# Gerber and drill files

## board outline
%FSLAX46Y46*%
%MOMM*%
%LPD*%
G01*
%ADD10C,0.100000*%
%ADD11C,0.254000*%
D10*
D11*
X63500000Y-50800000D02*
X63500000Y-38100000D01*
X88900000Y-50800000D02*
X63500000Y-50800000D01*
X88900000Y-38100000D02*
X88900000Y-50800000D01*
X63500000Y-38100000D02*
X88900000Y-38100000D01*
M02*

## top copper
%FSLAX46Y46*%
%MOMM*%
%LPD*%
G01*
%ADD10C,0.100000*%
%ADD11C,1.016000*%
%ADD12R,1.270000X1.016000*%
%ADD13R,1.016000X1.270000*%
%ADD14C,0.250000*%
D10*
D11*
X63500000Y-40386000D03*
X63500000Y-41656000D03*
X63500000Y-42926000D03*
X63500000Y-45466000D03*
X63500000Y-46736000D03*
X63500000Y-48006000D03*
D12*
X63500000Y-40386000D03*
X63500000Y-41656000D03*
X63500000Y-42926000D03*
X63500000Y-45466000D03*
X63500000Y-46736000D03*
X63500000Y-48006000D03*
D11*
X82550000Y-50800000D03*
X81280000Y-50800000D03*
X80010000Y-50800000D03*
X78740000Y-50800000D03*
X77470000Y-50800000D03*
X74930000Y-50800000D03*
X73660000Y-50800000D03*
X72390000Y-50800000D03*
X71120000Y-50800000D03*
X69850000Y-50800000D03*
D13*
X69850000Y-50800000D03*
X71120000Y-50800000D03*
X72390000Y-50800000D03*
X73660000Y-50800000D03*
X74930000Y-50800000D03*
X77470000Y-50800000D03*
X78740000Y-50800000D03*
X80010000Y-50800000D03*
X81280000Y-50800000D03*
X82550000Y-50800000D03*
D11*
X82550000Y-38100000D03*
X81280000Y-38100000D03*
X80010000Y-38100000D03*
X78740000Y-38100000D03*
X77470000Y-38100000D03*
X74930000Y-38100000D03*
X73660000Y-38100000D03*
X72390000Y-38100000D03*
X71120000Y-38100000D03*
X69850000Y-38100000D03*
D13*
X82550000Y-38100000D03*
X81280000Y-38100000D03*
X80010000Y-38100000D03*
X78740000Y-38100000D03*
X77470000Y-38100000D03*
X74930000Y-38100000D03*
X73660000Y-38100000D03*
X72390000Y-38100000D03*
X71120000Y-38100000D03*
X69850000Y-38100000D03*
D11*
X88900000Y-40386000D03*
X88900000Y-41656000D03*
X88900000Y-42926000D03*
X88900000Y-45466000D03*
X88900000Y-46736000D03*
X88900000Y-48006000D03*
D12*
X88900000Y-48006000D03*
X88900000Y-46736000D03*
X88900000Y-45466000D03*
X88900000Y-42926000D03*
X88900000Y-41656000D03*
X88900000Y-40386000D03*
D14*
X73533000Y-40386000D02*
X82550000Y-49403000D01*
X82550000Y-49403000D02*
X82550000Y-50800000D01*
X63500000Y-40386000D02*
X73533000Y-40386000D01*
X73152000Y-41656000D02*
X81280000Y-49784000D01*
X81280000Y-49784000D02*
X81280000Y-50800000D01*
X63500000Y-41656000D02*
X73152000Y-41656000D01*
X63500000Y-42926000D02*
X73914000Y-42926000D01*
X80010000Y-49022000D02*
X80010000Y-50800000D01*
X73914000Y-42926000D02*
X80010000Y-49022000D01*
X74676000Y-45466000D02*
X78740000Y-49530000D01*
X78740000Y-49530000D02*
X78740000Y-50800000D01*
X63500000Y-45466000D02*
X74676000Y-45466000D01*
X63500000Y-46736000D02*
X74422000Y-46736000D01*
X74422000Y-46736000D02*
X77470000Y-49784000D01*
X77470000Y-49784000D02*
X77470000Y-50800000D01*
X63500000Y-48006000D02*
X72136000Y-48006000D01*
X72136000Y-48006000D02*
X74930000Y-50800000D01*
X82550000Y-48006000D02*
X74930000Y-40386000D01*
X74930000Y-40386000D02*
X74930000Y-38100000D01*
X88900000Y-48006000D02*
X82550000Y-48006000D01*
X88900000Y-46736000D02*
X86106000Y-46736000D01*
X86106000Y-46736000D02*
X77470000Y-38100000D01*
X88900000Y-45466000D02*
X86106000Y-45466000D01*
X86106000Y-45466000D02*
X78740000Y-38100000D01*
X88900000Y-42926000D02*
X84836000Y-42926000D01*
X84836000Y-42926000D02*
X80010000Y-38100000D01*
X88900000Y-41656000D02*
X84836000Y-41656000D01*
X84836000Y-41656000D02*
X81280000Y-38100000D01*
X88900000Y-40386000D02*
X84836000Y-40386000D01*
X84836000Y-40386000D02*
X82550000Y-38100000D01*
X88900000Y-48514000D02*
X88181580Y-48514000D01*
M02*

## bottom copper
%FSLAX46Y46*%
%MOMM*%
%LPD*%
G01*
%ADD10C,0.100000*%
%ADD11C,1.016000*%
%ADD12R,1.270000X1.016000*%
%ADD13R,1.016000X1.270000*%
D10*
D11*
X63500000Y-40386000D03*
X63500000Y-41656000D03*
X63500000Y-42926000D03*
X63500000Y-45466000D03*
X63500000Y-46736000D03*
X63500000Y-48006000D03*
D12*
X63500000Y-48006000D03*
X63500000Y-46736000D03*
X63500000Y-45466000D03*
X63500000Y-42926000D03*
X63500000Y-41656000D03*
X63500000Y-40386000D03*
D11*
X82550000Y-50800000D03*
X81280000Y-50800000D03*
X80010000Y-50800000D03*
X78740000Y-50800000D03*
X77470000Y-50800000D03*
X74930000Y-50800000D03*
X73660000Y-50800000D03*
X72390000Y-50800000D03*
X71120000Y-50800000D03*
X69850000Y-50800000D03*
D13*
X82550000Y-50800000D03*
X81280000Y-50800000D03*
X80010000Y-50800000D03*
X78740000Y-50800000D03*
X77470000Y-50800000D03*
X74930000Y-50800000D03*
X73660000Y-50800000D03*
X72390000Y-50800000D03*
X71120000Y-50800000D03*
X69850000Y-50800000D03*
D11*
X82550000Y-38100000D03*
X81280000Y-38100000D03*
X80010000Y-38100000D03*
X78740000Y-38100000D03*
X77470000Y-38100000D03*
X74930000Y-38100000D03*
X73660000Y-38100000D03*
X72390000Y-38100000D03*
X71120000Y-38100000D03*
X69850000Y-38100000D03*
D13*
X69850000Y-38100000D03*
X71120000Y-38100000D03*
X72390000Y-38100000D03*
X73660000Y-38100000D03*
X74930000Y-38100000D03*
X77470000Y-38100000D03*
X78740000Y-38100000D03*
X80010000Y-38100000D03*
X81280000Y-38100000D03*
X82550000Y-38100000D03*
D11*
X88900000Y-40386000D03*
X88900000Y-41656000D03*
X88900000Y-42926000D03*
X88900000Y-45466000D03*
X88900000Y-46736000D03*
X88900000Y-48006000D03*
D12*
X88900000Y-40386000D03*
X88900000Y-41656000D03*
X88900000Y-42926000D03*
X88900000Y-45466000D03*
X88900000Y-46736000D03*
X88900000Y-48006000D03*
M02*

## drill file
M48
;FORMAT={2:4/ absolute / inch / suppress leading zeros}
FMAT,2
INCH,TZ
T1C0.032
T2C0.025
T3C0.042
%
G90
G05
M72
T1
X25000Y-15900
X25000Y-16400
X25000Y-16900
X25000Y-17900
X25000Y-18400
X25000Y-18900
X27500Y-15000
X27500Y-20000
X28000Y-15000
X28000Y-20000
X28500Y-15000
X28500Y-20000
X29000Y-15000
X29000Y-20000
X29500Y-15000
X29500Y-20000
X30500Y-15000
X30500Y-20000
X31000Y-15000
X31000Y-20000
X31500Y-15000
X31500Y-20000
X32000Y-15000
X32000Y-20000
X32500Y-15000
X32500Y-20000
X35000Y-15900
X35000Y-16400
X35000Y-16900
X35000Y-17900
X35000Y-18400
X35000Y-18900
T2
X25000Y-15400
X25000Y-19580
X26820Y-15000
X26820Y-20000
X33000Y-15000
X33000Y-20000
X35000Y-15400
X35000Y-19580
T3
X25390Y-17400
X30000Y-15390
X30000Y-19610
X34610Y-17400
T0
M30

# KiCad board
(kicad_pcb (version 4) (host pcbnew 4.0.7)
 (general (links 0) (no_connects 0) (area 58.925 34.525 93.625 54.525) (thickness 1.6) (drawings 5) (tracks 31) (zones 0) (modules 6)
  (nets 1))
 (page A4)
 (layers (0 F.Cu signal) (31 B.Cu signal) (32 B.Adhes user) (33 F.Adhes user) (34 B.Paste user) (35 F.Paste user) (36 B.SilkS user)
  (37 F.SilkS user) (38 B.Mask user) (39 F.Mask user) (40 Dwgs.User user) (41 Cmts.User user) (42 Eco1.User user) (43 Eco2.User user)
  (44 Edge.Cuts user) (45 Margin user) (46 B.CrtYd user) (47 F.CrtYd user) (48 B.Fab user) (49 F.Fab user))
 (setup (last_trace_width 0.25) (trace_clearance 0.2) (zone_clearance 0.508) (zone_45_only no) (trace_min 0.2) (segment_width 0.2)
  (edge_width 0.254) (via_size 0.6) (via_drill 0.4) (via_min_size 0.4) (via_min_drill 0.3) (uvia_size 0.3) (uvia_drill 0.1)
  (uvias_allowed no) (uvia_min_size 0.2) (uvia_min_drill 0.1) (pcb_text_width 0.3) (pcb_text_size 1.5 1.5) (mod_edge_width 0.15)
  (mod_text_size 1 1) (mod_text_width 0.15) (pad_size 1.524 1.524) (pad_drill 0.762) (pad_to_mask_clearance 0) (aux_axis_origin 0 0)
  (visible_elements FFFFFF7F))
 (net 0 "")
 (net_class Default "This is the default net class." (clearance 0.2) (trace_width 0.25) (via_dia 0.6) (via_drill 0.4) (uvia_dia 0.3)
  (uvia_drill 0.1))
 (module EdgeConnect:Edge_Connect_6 (layer F.Cu) (at 63.5 44.196 90)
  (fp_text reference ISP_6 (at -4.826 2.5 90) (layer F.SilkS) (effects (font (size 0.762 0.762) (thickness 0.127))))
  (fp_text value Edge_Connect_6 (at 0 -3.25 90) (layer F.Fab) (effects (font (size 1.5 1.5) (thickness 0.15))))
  (pad 1 thru_hole circle (at 3.81 0 90) (size 1.016 1.016) (drill 0.8128) (layers *.Cu *.Mask))
  (pad "" np_thru_hole circle (at 0 0.9906 90) (size 1.0668 1.0668) (drill 1.0668) (layers *.Cu))
  (pad 2 thru_hole circle (at 2.54 0 90) (size 1.016 1.016) (drill 0.8128) (layers *.Cu *.Mask))
  (pad 3 thru_hole circle (at 1.27 0 90) (size 1.016 1.016) (drill 0.8128) (layers *.Cu *.Mask))
  (pad 4 thru_hole circle (at -1.27 0 90) (size 1.016 1.016) (drill 0.8128) (layers *.Cu *.Mask))
  (pad 5 thru_hole circle (at -2.54 0 90) (size 1.016 1.016) (drill 0.8128) (layers *.Cu *.Mask))
  (pad 6 thru_hole circle (at -3.81 0 90) (size 1.016 1.016) (drill 0.8128) (layers *.Cu *.Mask))
  (pad "" np_thru_hole circle (at -5.5372 0 90) (size 0.635 0.635) (drill 0.635) (layers *.Cu))
  (pad "" np_thru_hole circle (at 5.08 0 90) (size 0.635 0.635) (drill 0.635) (layers *.Cu))
  (pad 1 smd rect (at 3.81 0 90) (size 1.016 1.27) (layers F.Cu F.Mask))
  (pad 2 smd rect (at 2.54 0 90) (size 1.016 1.27) (layers F.Cu F.Mask))
  (pad 3 smd rect (at 1.27 0 90) (size 1.016 1.27) (layers F.Cu F.Mask))
  (pad 4 smd rect (at -1.27 0 90) (size 1.016 1.27) (layers F.Cu F.Mask))
  (pad 5 smd rect (at -2.54 0 90) (size 1.016 1.27) (layers F.Cu F.Mask))
  (pad 6 smd rect (at -3.81 0 90) (size 1.016 1.27) (layers F.Cu F.Mask))
  (pad 6 smd rect (at -3.81 0 90) (size 1.016 1.27) (layers B.Cu B.Mask))
  (pad 5 smd rect (at -2.54 0 90) (size 1.016 1.27) (layers B.Cu B.Mask))
  (pad 4 smd rect (at -1.27 0 90) (size 1.016 1.27) (layers B.Cu B.Mask))
  (pad 3 smd rect (at 1.27 0 90) (size 1.016 1.27) (layers B.Cu B.Mask))
  (pad 2 smd rect (at 2.54 0 90) (size 1.016 1.27) (layers B.Cu B.Mask))
  (pad 1 smd rect (at 3.81 0 90) (size 1.016 1.27) (layers B.Cu B.Mask)))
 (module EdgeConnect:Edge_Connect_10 (layer B.Cu) (at 76.2 50.8)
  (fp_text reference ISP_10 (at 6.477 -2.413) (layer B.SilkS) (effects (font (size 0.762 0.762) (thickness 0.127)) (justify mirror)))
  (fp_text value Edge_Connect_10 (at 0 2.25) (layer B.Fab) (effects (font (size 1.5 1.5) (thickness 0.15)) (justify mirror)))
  (pad 1 thru_hole circle (at 6.35 0) (size 1.016 1.016) (drill 0.8128) (layers *.Cu *.Mask))
  (pad "" np_thru_hole circle (at 0 -0.9906) (size 1.0668 1.0668) (drill 1.0668) (layers *.Cu))
  (pad 2 thru_hole circle (at 5.08 0) (size 1.016 1.016) (drill 0.8128) (layers *.Cu *.Mask))
  (pad 3 thru_hole circle (at 3.81 0) (size 1.016 1.016) (drill 0.8128) (layers *.Cu *.Mask))
  (pad 4 thru_hole circle (at 2.54 0) (size 1.016 1.016) (drill 0.8128) (layers *.Cu *.Mask))
  (pad 5 thru_hole circle (at 1.27 0) (size 1.016 1.016) (drill 0.8128) (layers *.Cu *.Mask))
  (pad 6 thru_hole circle (at -1.27 0) (size 1.016 1.016) (drill 0.8128) (layers *.Cu *.Mask))
  (pad "" np_thru_hole circle (at -8.0772 0) (size 0.635 0.635) (drill 0.635) (layers *.Cu))
  (pad "" np_thru_hole circle (at 7.62 0) (size 0.635 0.635) (drill 0.635) (layers *.Cu))
  (pad 7 thru_hole circle (at -2.54 0) (size 1.016 1.016) (drill 0.8128) (layers *.Cu *.Mask))
  (pad 8 thru_hole circle (at -3.81 0) (size 1.016 1.016) (drill 0.8128) (layers *.Cu *.Mask))
  (pad 9 thru_hole circle (at -5.08 0) (size 1.016 1.016) (drill 0.8128) (layers *.Cu *.Mask))
  (pad 10 thru_hole circle (at -6.35 0) (size 1.016 1.016) (drill 0.8128) (layers *.Cu *.Mask))
  (pad 1 smd rect (at 6.35 0) (size 1.016 1.27) (layers B.Cu B.Mask))
  (pad 2 smd rect (at 5.08 0) (size 1.016 1.27) (layers B.Cu B.Mask))
  (pad 3 smd rect (at 3.81 0) (size 1.016 1.27) (layers B.Cu B.Mask))
  (pad 4 smd rect (at 2.54 0) (size 1.016 1.27) (layers B.Cu B.Mask))
  (pad 5 smd rect (at 1.27 0) (size 1.016 1.27) (layers B.Cu B.Mask))
  (pad 5 smd rect (at -1.27 0) (size 1.016 1.27) (layers B.Cu B.Mask))
  (pad 7 smd rect (at -2.54 0) (size 1.016 1.27) (layers B.Cu B.Mask))
  (pad 8 smd rect (at -3.81 0) (size 1.016 1.27) (layers B.Cu B.Mask))
  (pad 9 smd rect (at -5.08 0) (size 1.016 1.27) (layers B.Cu B.Mask))
  (pad 10 smd rect (at -6.35 0) (size 1.016 1.27) (layers B.Cu B.Mask))
  (pad 10 smd rect (at -6.35 0) (size 1.016 1.27) (layers F.Cu F.Mask))
  (pad 9 smd rect (at -5.08 0) (size 1.016 1.27) (layers F.Cu F.Mask))
  (pad 8 smd rect (at -3.81 0) (size 1.016 1.27) (layers F.Cu F.Mask))
  (pad 7 smd rect (at -2.54 0) (size 1.016 1.27) (layers F.Cu F.Mask))
  (pad 5 smd rect (at -1.27 0) (size 1.016 1.27) (layers F.Cu F.Mask))
  (pad 5 smd rect (at 1.27 0) (size 1.016 1.27) (layers F.Cu F.Mask))
  (pad 4 smd rect (at 2.54 0) (size 1.016 1.27) (layers F.Cu F.Mask))
  (pad 3 smd rect (at 3.81 0) (size 1.016 1.27) (layers F.Cu F.Mask))
  (pad 2 smd rect (at 5.08 0) (size 1.016 1.27) (layers F.Cu F.Mask))
  (pad 1 smd rect (at 6.35 0) (size 1.016 1.27) (layers F.Cu F.Mask)))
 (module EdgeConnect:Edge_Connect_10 (layer F.Cu) (at 76.2 38.1)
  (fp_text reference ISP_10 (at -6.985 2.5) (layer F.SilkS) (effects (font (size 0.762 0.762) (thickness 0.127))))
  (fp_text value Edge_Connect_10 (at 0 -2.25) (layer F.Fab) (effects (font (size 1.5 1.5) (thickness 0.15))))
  (pad 1 thru_hole circle (at 6.35 0) (size 1.016 1.016) (drill 0.8128) (layers *.Cu *.Mask))
  (pad "" np_thru_hole circle (at 0 0.9906) (size 1.0668 1.0668) (drill 1.0668) (layers *.Cu))
  (pad 2 thru_hole circle (at 5.08 0) (size 1.016 1.016) (drill 0.8128) (layers *.Cu *.Mask))
  (pad 3 thru_hole circle (at 3.81 0) (size 1.016 1.016) (drill 0.8128) (layers *.Cu *.Mask))
  (pad 4 thru_hole circle (at 2.54 0) (size 1.016 1.016) (drill 0.8128) (layers *.Cu *.Mask))
  (pad 5 thru_hole circle (at 1.27 0) (size 1.016 1.016) (drill 0.8128) (layers *.Cu *.Mask))
  (pad 6 thru_hole circle (at -1.27 0) (size 1.016 1.016) (drill 0.8128) (layers *.Cu *.Mask))
  (pad "" np_thru_hole circle (at -8.0772 0) (size 0.635 0.635) (drill 0.635) (layers *.Cu))
  (pad "" np_thru_hole circle (at 7.62 0) (size 0.635 0.635) (drill 0.635) (layers *.Cu))
  (pad 7 thru_hole circle (at -2.54 0) (size 1.016 1.016) (drill 0.8128) (layers *.Cu *.Mask))
  (pad 8 thru_hole circle (at -3.81 0) (size 1.016 1.016) (drill 0.8128) (layers *.Cu *.Mask))
  (pad 9 thru_hole circle (at -5.08 0) (size 1.016 1.016) (drill 0.8128) (layers *.Cu *.Mask))
  (pad 10 thru_hole circle (at -6.35 0) (size 1.016 1.016) (drill 0.8128) (layers *.Cu *.Mask))
  (pad 1 smd rect (at 6.35 0) (size 1.016 1.27) (layers F.Cu F.Mask))
  (pad 2 smd rect (at 5.08 0) (size 1.016 1.27) (layers F.Cu F.Mask))
  (pad 3 smd rect (at 3.81 0) (size 1.016 1.27) (layers F.Cu F.Mask))
  (pad 4 smd rect (at 2.54 0) (size 1.016 1.27) (layers F.Cu F.Mask))
  (pad 5 smd rect (at 1.27 0) (size 1.016 1.27) (layers F.Cu F.Mask))
  (pad 5 smd rect (at -1.27 0) (size 1.016 1.27) (layers F.Cu F.Mask))
  (pad 7 smd rect (at -2.54 0) (size 1.016 1.27) (layers F.Cu F.Mask))
  (pad 8 smd rect (at -3.81 0) (size 1.016 1.27) (layers F.Cu F.Mask))
  (pad 9 smd rect (at -5.08 0) (size 1.016 1.27) (layers F.Cu F.Mask))
  (pad 10 smd rect (at -6.35 0) (size 1.016 1.27) (layers F.Cu F.Mask))
  (pad 10 smd rect (at -6.35 0) (size 1.016 1.27) (layers B.Cu B.Mask))
  (pad 9 smd rect (at -5.08 0) (size 1.016 1.27) (layers B.Cu B.Mask))
  (pad 8 smd rect (at -3.81 0) (size 1.016 1.27) (layers B.Cu B.Mask))
  (pad 7 smd rect (at -2.54 0) (size 1.016 1.27) (layers B.Cu B.Mask))
  (pad 5 smd rect (at -1.27 0) (size 1.016 1.27) (layers B.Cu B.Mask))
  (pad 5 smd rect (at 1.27 0) (size 1.016 1.27) (layers B.Cu B.Mask))
  (pad 4 smd rect (at 2.54 0) (size 1.016 1.27) (layers B.Cu B.Mask))
  (pad 3 smd rect (at 3.81 0) (size 1.016 1.27) (layers B.Cu B.Mask))
  (pad 2 smd rect (at 5.08 0) (size 1.016 1.27) (layers B.Cu B.Mask))
  (pad 1 smd rect (at 6.35 0) (size 1.016 1.27) (layers B.Cu B.Mask)))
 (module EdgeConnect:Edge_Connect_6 (layer B.Cu) (at 88.9 44.196 90)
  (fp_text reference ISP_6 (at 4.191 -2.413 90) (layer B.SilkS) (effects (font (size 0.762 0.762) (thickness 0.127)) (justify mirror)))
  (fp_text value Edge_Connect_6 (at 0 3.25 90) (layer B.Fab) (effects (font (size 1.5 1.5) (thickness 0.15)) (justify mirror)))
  (pad 1 thru_hole circle (at 3.81 0 90) (size 1.016 1.016) (drill 0.8128) (layers *.Cu *.Mask))
  (pad "" np_thru_hole circle (at 0 -0.9906 90) (size 1.0668 1.0668) (drill 1.0668) (layers *.Cu))
  (pad 2 thru_hole circle (at 2.54 0 90) (size 1.016 1.016) (drill 0.8128) (layers *.Cu *.Mask))
  (pad 3 thru_hole circle (at 1.27 0 90) (size 1.016 1.016) (drill 0.8128) (layers *.Cu *.Mask))
  (pad 4 thru_hole circle (at -1.27 0 90) (size 1.016 1.016) (drill 0.8128) (layers *.Cu *.Mask))
  (pad 5 thru_hole circle (at -2.54 0 90) (size 1.016 1.016) (drill 0.8128) (layers *.Cu *.Mask))
  (pad 6 thru_hole circle (at -3.81 0 90) (size 1.016 1.016) (drill 0.8128) (layers *.Cu *.Mask))
  (pad "" np_thru_hole circle (at -5.5372 0 90) (size 0.635 0.635) (drill 0.635) (layers *.Cu))
  (pad "" np_thru_hole circle (at 5.08 0 90) (size 0.635 0.635) (drill 0.635) (layers *.Cu))
  (pad 1 smd rect (at 3.81 0 90) (size 1.016 1.27) (layers B.Cu B.Mask))
  (pad 2 smd rect (at 2.54 0 90) (size 1.016 1.27) (layers B.Cu B.Mask))
  (pad 3 smd rect (at 1.27 0 90) (size 1.016 1.27) (layers B.Cu B.Mask))
  (pad 4 smd rect (at -1.27 0 90) (size 1.016 1.27) (layers B.Cu B.Mask))
  (pad 5 smd rect (at -2.54 0 90) (size 1.016 1.27) (layers B.Cu B.Mask))
  (pad 6 smd rect (at -3.81 0 90) (size 1.016 1.27) (layers B.Cu B.Mask))
  (pad 6 smd rect (at -3.81 0 90) (size 1.016 1.27) (layers F.Cu F.Mask))
  (pad 5 smd rect (at -2.54 0 90) (size 1.016 1.27) (layers F.Cu F.Mask))
  (pad 4 smd rect (at -1.27 0 90) (size 1.016 1.27) (layers F.Cu F.Mask))
  (pad 3 smd rect (at 1.27 0 90) (size 1.016 1.27) (layers F.Cu F.Mask))
  (pad 2 smd rect (at 2.54 0 90) (size 1.016 1.27) (layers F.Cu F.Mask))
  (pad 1 smd rect (at 3.81 0 90) (size 1.016 1.27) (layers F.Cu F.Mask)))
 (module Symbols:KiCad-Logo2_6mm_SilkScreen (layer B.Cu) (at 76.2 44.45 180)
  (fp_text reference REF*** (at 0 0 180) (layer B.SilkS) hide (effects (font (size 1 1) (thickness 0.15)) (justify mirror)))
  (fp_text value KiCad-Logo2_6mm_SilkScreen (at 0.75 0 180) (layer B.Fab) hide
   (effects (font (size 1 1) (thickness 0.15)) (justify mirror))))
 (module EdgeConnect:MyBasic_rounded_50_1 (layer F.Cu) (at 76.2 46.736)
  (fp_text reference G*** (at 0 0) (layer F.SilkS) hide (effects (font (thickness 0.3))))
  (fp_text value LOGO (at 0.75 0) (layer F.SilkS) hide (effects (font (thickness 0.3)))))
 (gr_line (start 63.5 50.8) (end 63.5 38.1) (layer Edge.Cuts) (width 0.254))
 (gr_line (start 88.9 50.8) (end 63.5 50.8) (layer Edge.Cuts) (width 0.254))
 (gr_line (start 88.9 38.1) (end 88.9 50.8) (layer Edge.Cuts) (width 0.254))
 (gr_line (start 63.5 38.1) (end 88.9 38.1) (layer Edge.Cuts) (width 0.254))
 (segment (start 73.533 40.386) (end 82.55 49.403) (width 0.25) (layer F.Cu) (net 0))
 (segment (start 82.55 49.403) (end 82.55 50.8) (width 0.25) (layer F.Cu) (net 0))
 (segment (start 63.5 40.386) (end 73.533 40.386) (width 0.25) (layer F.Cu) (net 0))
 (segment (start 73.152 41.656) (end 81.28 49.784) (width 0.25) (layer F.Cu) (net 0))
 (segment (start 81.28 49.784) (end 81.28 50.8) (width 0.25) (layer F.Cu) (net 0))
 (segment (start 63.5 41.656) (end 73.152 41.656) (width 0.25) (layer F.Cu) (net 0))
 (segment (start 63.5 42.926) (end 73.914 42.926) (width 0.25) (layer F.Cu) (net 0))
 (segment (start 80.01 49.022) (end 80.01 50.8) (width 0.25) (layer F.Cu) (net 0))
 (segment (start 73.914 42.926) (end 80.01 49.022) (width 0.25) (layer F.Cu) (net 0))
 (segment (start 74.676 45.466) (end 78.74 49.53) (width 0.25) (layer F.Cu) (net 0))
 (segment (start 78.74 49.53) (end 78.74 50.8) (width 0.25) (layer F.Cu) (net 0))
 (segment (start 63.5 45.466) (end 74.676 45.466) (width 0.25) (layer F.Cu) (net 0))
 (segment (start 63.5 46.736) (end 74.422 46.736) (width 0.25) (layer F.Cu) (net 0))
 (segment (start 74.422 46.736) (end 77.47 49.784) (width 0.25) (layer F.Cu) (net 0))
 (segment (start 77.47 49.784) (end 77.47 50.8) (width 0.25) (layer F.Cu) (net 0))
 (segment (start 63.5 48.006) (end 72.136 48.006) (width 0.25) (layer F.Cu) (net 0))
 (segment (start 72.136 48.006) (end 74.93 50.8) (width 0.25) (layer F.Cu) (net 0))
 (segment (start 82.55 48.006) (end 74.93 40.386) (width 0.25) (layer F.Cu) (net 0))
 (segment (start 74.93 40.386) (end 74.93 38.1) (width 0.25) (layer F.Cu) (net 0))
 (segment (start 88.9 48.006) (end 82.55 48.006) (width 0.25) (layer F.Cu) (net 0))
 (segment (start 88.9 46.736) (end 86.106 46.736) (width 0.25) (layer F.Cu) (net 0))
 (segment (start 86.106 46.736) (end 77.47 38.1) (width 0.25) (layer F.Cu) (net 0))
 (segment (start 88.9 45.466) (end 86.106 45.466) (width 0.25) (layer F.Cu) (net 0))
 (segment (start 86.106 45.466) (end 78.74 38.1) (width 0.25) (layer F.Cu) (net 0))
 (segment (start 88.9 42.926) (end 84.836 42.926) (width 0.25) (layer F.Cu) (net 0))
 (segment (start 84.836 42.926) (end 80.01 38.1) (width 0.25) (layer F.Cu) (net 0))
 (segment (start 88.9 41.656) (end 84.836 41.656) (width 0.25) (layer F.Cu) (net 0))
 (segment (start 84.836 41.656) (end 81.28 38.1) (width 0.25) (layer F.Cu) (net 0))
 (segment (start 88.9 40.386) (end 84.836 40.386) (width 0.25) (layer F.Cu) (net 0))
 (segment (start 84.836 40.386) (end 82.55 38.1) (width 0.25) (layer F.Cu) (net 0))
 (segment (start 88.9 48.514) (end 88.18158 48.514) (width 0.25) (layer F.Cu) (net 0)))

